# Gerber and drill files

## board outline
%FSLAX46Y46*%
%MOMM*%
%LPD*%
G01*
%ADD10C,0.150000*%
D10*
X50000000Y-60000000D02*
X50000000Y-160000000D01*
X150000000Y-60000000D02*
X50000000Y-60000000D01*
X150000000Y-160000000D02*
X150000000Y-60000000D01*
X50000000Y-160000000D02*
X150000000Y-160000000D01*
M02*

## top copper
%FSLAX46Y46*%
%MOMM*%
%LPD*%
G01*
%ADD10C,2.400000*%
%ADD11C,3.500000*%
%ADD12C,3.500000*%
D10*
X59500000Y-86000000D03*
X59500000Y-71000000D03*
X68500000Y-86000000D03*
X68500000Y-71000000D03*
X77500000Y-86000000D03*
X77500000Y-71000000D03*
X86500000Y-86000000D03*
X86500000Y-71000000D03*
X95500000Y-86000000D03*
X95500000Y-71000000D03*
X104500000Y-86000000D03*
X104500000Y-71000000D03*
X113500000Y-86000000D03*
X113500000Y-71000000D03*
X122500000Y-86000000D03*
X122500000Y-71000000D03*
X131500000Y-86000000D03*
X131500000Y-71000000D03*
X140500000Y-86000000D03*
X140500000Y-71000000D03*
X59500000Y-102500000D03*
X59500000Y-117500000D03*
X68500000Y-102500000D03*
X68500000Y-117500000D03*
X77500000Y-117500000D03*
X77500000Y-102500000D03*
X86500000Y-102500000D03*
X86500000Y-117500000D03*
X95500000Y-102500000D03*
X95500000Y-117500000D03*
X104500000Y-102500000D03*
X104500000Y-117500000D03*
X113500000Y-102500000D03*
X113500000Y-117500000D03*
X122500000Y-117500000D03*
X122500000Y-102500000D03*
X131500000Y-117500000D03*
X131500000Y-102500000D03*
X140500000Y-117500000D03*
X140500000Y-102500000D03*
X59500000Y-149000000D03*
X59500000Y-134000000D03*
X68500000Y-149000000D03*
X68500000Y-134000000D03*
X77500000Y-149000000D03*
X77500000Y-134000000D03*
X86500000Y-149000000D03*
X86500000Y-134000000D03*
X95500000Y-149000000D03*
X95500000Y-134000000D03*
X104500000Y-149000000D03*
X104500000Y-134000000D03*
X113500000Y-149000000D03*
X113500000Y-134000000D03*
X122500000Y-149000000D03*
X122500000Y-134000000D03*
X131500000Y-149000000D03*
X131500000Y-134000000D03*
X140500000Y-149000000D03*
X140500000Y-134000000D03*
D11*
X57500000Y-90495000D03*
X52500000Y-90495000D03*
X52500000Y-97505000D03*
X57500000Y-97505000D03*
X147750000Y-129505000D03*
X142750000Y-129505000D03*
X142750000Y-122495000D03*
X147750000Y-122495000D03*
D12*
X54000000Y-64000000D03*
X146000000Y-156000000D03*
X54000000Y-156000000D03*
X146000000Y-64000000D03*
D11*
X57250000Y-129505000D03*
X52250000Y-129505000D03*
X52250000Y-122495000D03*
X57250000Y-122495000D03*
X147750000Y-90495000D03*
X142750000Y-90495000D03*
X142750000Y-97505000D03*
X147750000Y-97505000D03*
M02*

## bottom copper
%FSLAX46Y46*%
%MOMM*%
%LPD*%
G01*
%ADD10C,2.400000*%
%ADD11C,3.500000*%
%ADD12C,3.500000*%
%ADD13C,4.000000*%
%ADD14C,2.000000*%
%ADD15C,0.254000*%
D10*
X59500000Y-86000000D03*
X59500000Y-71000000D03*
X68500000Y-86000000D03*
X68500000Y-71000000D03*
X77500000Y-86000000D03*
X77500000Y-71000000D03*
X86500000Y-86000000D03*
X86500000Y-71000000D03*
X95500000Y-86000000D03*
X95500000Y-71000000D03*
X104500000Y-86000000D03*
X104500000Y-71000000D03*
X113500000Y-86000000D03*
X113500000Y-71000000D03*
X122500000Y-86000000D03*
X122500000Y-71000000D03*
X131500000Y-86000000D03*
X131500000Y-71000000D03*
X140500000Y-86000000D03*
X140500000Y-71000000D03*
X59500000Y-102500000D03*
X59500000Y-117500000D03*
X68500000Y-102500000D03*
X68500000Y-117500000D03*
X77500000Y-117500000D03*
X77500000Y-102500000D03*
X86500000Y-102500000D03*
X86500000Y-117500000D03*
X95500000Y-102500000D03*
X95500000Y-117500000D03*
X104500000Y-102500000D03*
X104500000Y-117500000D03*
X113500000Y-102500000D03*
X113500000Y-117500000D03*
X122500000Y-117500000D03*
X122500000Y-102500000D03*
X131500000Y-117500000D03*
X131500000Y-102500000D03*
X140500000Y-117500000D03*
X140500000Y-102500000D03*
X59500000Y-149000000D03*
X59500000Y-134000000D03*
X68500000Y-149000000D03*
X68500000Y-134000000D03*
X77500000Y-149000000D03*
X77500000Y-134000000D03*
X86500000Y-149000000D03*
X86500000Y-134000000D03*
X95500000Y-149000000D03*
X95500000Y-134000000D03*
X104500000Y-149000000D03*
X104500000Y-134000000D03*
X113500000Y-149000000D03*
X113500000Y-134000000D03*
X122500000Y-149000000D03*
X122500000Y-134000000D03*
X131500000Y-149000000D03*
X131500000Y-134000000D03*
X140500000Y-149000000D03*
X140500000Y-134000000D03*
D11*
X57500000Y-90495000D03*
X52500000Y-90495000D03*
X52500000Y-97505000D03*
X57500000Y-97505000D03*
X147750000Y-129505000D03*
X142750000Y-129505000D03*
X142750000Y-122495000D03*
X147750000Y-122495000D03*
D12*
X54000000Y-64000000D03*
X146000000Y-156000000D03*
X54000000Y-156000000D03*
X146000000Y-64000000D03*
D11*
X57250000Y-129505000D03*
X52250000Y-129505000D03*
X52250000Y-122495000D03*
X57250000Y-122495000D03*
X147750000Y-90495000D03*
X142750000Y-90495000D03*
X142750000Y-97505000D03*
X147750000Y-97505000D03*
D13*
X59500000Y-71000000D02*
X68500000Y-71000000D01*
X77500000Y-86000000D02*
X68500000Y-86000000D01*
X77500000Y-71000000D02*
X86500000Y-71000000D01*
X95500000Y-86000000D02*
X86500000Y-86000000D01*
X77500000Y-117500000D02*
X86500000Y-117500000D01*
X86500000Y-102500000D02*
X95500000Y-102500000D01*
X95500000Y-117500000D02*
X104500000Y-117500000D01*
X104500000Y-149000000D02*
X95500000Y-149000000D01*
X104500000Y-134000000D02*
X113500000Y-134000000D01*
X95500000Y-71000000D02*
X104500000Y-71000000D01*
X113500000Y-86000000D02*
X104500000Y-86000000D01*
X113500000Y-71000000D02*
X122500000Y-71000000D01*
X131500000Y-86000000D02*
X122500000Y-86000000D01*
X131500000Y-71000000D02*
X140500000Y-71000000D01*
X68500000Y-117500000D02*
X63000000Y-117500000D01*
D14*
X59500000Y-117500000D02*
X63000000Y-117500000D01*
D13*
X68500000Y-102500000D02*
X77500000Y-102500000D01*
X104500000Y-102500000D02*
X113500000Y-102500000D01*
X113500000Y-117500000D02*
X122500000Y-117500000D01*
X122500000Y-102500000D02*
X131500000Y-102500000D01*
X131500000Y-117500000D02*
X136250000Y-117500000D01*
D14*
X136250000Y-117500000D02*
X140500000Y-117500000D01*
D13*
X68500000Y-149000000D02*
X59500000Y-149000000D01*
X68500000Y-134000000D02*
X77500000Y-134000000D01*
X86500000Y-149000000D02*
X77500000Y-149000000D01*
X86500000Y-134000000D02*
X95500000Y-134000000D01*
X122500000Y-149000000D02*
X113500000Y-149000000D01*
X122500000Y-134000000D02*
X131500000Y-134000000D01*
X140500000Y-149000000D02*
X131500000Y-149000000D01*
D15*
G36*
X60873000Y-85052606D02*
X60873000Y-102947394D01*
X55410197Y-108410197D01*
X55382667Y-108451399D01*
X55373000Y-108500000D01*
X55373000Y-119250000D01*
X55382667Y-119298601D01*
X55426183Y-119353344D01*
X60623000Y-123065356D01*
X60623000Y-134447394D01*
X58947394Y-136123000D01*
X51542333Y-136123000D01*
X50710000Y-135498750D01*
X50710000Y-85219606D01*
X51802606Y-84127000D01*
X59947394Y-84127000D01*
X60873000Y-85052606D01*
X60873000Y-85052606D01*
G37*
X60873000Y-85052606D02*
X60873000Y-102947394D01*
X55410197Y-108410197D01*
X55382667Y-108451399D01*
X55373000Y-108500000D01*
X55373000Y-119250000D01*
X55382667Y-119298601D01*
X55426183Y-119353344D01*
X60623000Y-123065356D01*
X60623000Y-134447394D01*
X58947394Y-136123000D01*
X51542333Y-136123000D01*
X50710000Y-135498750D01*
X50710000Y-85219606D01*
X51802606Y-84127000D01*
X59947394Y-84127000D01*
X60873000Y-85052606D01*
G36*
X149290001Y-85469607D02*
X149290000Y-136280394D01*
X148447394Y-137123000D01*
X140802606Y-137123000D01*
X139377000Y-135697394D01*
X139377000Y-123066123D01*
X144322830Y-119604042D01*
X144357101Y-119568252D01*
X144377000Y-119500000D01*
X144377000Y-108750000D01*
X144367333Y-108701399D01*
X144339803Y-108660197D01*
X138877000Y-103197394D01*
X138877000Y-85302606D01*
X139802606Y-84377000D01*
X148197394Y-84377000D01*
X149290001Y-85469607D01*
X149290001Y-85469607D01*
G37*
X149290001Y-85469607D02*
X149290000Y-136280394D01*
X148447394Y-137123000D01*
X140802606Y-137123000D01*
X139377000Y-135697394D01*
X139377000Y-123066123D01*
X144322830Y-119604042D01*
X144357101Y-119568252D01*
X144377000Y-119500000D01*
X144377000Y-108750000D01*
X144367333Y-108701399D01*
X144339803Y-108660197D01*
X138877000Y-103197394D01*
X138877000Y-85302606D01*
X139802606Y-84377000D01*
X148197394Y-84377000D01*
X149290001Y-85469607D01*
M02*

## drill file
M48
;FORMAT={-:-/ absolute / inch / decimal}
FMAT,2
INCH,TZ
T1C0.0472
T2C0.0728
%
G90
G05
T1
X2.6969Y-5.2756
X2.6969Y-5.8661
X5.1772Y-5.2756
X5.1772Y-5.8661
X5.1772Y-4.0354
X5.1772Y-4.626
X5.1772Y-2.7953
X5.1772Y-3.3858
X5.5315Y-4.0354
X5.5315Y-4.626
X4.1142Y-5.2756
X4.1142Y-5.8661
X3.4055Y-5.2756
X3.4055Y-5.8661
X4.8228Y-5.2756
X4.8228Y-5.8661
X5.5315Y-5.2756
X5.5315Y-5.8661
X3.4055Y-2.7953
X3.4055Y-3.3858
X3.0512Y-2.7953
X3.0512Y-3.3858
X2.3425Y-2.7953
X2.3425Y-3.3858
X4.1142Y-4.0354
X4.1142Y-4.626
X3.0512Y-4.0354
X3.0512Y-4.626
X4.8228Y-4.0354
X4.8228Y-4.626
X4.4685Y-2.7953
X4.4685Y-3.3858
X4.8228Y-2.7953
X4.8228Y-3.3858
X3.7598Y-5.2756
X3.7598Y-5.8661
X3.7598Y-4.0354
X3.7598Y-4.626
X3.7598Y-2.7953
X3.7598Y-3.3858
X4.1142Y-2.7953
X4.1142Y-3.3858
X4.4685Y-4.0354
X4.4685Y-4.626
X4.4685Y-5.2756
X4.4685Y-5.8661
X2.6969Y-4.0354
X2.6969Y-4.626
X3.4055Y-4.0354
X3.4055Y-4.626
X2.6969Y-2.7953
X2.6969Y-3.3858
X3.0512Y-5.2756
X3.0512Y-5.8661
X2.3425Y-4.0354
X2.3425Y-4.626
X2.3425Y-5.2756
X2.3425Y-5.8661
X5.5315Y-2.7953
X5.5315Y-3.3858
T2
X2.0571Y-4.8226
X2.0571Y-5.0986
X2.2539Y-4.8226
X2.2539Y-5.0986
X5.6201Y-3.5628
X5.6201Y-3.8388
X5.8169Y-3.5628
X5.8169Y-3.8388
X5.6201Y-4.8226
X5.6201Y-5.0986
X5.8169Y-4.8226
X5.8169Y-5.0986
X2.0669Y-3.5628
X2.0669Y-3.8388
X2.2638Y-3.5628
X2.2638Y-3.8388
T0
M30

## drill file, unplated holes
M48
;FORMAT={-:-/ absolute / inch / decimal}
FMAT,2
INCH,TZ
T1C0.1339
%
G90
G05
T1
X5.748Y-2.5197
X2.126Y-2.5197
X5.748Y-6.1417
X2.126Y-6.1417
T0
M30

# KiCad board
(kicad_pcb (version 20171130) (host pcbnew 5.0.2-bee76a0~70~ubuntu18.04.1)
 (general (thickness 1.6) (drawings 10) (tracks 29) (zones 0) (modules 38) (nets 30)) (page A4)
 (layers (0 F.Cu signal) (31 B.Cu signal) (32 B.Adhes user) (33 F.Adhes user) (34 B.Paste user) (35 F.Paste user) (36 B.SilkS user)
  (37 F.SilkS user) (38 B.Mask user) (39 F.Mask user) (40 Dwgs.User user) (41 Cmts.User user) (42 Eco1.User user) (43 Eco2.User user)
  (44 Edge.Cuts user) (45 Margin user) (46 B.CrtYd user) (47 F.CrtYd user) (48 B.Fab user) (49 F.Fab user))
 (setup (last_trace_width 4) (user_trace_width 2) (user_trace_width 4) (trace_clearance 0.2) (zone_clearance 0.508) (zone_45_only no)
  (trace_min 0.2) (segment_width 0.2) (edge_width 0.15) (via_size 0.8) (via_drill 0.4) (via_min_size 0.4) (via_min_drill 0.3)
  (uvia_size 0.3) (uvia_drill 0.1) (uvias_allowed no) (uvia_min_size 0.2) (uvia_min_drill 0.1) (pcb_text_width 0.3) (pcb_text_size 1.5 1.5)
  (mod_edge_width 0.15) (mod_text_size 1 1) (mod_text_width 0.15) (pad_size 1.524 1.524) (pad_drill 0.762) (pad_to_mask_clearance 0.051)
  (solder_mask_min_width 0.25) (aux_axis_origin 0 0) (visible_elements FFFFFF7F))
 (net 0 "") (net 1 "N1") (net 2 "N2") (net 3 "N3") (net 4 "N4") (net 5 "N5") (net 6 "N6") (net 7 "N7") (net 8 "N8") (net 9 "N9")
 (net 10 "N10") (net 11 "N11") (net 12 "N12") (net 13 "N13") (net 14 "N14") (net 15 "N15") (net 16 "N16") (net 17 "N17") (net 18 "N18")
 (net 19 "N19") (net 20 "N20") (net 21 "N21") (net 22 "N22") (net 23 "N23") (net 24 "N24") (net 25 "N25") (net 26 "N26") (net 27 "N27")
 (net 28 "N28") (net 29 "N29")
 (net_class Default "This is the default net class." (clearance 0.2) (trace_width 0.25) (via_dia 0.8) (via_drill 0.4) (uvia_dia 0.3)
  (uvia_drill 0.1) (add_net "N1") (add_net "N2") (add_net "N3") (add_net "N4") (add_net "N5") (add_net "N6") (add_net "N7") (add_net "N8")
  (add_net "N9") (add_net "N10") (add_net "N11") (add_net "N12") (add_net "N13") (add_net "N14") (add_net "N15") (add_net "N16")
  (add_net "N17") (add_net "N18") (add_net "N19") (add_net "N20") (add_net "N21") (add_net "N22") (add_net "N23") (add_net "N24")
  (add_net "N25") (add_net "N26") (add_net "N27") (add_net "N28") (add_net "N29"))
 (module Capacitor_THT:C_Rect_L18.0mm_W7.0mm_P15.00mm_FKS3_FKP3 (layer F.Cu) (at 59.5 86 90)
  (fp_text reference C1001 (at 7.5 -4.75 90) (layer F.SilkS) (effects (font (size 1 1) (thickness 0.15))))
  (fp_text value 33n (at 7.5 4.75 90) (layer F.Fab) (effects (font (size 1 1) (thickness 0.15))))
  (pad 1 thru_hole circle (at 0 0 90) (size 2.4 2.4) (drill 1.2) (layers *.Cu *.Mask) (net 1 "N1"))
  (pad 2 thru_hole circle (at 15 0 90) (size 2.4 2.4) (drill 1.2) (layers *.Cu *.Mask) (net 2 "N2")))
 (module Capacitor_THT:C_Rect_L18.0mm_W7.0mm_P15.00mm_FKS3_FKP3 (layer F.Cu) (at 68.5 71 270)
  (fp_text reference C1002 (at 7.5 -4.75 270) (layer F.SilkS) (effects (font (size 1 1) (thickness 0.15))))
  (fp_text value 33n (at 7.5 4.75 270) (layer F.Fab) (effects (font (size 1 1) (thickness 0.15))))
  (pad 2 thru_hole circle (at 15 0 270) (size 2.4 2.4) (drill 1.2) (layers *.Cu *.Mask) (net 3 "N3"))
  (pad 1 thru_hole circle (at 0 0 270) (size 2.4 2.4) (drill 1.2) (layers *.Cu *.Mask) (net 2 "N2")))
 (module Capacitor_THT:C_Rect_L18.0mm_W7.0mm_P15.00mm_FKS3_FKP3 (layer F.Cu) (at 77.5 86 90)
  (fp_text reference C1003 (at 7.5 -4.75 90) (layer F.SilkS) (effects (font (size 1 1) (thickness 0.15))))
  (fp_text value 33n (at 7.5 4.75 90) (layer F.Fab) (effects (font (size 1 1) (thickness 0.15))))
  (pad 1 thru_hole circle (at 0 0 90) (size 2.4 2.4) (drill 1.2) (layers *.Cu *.Mask) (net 3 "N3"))
  (pad 2 thru_hole circle (at 15 0 90) (size 2.4 2.4) (drill 1.2) (layers *.Cu *.Mask) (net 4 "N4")))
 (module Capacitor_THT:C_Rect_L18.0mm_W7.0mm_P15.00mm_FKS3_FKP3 (layer F.Cu) (at 86.5 71 270)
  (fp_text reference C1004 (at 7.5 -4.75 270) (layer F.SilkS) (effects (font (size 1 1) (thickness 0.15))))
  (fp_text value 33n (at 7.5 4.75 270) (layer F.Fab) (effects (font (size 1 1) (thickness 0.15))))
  (pad 2 thru_hole circle (at 15 0 270) (size 2.4 2.4) (drill 1.2) (layers *.Cu *.Mask) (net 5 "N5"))
  (pad 1 thru_hole circle (at 0 0 270) (size 2.4 2.4) (drill 1.2) (layers *.Cu *.Mask) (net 4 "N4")))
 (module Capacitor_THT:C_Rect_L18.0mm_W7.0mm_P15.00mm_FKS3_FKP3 (layer F.Cu) (at 95.5 86 90)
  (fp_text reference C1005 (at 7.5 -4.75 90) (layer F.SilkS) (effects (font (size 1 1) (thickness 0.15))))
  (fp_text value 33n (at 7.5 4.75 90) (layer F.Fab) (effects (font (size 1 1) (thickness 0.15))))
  (pad 1 thru_hole circle (at 0 0 90) (size 2.4 2.4) (drill 1.2) (layers *.Cu *.Mask) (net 5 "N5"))
  (pad 2 thru_hole circle (at 15 0 90) (size 2.4 2.4) (drill 1.2) (layers *.Cu *.Mask) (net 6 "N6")))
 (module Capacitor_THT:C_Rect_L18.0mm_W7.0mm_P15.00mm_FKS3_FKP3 (layer F.Cu) (at 104.5 71 270)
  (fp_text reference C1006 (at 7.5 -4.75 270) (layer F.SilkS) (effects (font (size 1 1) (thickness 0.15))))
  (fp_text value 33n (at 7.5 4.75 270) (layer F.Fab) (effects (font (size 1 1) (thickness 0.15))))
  (pad 2 thru_hole circle (at 15 0 270) (size 2.4 2.4) (drill 1.2) (layers *.Cu *.Mask) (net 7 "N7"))
  (pad 1 thru_hole circle (at 0 0 270) (size 2.4 2.4) (drill 1.2) (layers *.Cu *.Mask) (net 6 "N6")))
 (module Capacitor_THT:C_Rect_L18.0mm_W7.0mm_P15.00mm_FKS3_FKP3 (layer F.Cu) (at 113.5 86 90)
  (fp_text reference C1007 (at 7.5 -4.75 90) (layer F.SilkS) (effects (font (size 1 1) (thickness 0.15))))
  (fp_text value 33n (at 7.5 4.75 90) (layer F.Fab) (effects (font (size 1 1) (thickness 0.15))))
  (pad 1 thru_hole circle (at 0 0 90) (size 2.4 2.4) (drill 1.2) (layers *.Cu *.Mask) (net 7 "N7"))
  (pad 2 thru_hole circle (at 15 0 90) (size 2.4 2.4) (drill 1.2) (layers *.Cu *.Mask) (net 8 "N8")))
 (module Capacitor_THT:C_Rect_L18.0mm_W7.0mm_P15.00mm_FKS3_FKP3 (layer F.Cu) (at 122.5 71 270)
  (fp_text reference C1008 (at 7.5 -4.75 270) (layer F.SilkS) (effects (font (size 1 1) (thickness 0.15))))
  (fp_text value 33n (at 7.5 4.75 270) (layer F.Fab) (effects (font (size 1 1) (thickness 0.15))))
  (pad 2 thru_hole circle (at 15 0 270) (size 2.4 2.4) (drill 1.2) (layers *.Cu *.Mask) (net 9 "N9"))
  (pad 1 thru_hole circle (at 0 0 270) (size 2.4 2.4) (drill 1.2) (layers *.Cu *.Mask) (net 8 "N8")))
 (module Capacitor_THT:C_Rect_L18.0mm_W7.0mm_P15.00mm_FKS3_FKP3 (layer F.Cu) (at 131.5 86 90)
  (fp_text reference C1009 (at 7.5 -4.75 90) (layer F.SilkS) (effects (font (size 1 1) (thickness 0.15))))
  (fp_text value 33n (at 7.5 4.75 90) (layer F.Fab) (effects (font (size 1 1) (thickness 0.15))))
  (pad 1 thru_hole circle (at 0 0 90) (size 2.4 2.4) (drill 1.2) (layers *.Cu *.Mask) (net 9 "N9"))
  (pad 2 thru_hole circle (at 15 0 90) (size 2.4 2.4) (drill 1.2) (layers *.Cu *.Mask) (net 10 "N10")))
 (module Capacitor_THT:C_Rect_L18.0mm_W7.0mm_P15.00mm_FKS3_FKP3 (layer F.Cu) (at 140.5 71 270)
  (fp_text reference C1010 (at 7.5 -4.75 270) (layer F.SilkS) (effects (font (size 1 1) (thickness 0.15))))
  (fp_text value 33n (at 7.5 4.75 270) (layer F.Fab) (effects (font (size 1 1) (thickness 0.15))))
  (pad 2 thru_hole circle (at 15 0 270) (size 2.4 2.4) (drill 1.2) (layers *.Cu *.Mask) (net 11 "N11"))
  (pad 1 thru_hole circle (at 0 0 270) (size 2.4 2.4) (drill 1.2) (layers *.Cu *.Mask) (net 10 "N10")))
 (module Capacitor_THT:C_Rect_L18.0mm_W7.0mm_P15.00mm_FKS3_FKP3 (layer F.Cu) (at 59.5 102.5 270)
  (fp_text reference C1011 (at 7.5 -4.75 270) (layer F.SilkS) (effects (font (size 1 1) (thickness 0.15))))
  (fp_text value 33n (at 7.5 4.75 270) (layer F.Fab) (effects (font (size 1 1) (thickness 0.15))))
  (pad 1 thru_hole circle (at 0 0 270) (size 2.4 2.4) (drill 1.2) (layers *.Cu *.Mask) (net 1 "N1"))
  (pad 2 thru_hole circle (at 15 0 270) (size 2.4 2.4) (drill 1.2) (layers *.Cu *.Mask) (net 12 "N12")))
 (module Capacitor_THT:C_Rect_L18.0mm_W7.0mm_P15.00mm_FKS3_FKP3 (layer F.Cu) (at 68.5 117.5 90)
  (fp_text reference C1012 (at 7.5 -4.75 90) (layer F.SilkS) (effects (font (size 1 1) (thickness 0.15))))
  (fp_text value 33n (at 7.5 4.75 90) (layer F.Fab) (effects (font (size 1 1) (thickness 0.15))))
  (pad 2 thru_hole circle (at 15 0 90) (size 2.4 2.4) (drill 1.2) (layers *.Cu *.Mask) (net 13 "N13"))
  (pad 1 thru_hole circle (at 0 0 90) (size 2.4 2.4) (drill 1.2) (layers *.Cu *.Mask) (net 12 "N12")))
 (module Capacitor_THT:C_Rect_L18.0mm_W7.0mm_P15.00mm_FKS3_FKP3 (layer F.Cu) (at 77.5 102.5 270)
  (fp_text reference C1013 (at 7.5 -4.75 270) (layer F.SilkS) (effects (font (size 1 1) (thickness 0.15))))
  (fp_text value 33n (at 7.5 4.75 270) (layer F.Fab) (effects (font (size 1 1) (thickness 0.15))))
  (pad 2 thru_hole circle (at 15 0 270) (size 2.4 2.4) (drill 1.2) (layers *.Cu *.Mask) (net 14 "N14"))
  (pad 1 thru_hole circle (at 0 0 270) (size 2.4 2.4) (drill 1.2) (layers *.Cu *.Mask) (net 13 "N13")))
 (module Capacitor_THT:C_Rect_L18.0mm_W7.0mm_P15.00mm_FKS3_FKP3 (layer F.Cu) (at 86.5 117.5 90)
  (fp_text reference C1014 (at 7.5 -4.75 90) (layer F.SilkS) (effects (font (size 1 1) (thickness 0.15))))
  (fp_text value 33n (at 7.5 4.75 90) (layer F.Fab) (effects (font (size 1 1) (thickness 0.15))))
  (pad 2 thru_hole circle (at 15 0 90) (size 2.4 2.4) (drill 1.2) (layers *.Cu *.Mask) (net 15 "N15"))
  (pad 1 thru_hole circle (at 0 0 90) (size 2.4 2.4) (drill 1.2) (layers *.Cu *.Mask) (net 14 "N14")))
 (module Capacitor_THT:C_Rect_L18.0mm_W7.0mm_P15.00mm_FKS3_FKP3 (layer F.Cu) (at 95.5 102.5 270)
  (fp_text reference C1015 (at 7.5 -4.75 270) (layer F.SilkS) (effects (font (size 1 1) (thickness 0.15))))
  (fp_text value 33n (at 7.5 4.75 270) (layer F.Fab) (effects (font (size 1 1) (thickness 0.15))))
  (pad 1 thru_hole circle (at 0 0 270) (size 2.4 2.4) (drill 1.2) (layers *.Cu *.Mask) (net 15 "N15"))
  (pad 2 thru_hole circle (at 15 0 270) (size 2.4 2.4) (drill 1.2) (layers *.Cu *.Mask) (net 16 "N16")))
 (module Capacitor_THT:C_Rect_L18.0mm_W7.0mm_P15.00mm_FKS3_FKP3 (layer F.Cu) (at 104.5 117.5 90)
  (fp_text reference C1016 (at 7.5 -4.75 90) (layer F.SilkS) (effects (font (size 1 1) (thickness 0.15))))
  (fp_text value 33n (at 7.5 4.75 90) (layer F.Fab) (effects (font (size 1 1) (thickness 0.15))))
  (pad 2 thru_hole circle (at 15 0 90) (size 2.4 2.4) (drill 1.2) (layers *.Cu *.Mask) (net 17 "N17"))
  (pad 1 thru_hole circle (at 0 0 90) (size 2.4 2.4) (drill 1.2) (layers *.Cu *.Mask) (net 16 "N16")))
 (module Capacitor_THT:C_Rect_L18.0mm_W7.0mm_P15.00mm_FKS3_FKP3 (layer F.Cu) (at 113.5 102.5 270)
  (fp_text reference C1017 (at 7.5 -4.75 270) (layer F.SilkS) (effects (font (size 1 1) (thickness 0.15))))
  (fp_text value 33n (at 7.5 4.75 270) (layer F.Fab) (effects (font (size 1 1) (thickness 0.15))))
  (pad 1 thru_hole circle (at 0 0 270) (size 2.4 2.4) (drill 1.2) (layers *.Cu *.Mask) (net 17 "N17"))
  (pad 2 thru_hole circle (at 15 0 270) (size 2.4 2.4) (drill 1.2) (layers *.Cu *.Mask) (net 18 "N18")))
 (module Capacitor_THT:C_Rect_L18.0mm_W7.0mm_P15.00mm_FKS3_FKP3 (layer F.Cu) (at 122.5 117.5 90)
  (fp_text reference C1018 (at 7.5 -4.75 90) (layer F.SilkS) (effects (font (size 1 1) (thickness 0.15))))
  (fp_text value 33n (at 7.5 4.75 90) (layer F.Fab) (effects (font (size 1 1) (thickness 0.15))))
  (pad 1 thru_hole circle (at 0 0 90) (size 2.4 2.4) (drill 1.2) (layers *.Cu *.Mask) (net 18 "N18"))
  (pad 2 thru_hole circle (at 15 0 90) (size 2.4 2.4) (drill 1.2) (layers *.Cu *.Mask) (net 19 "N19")))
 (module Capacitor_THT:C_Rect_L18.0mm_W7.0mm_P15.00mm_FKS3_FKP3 (layer F.Cu) (at 131.5 102.5 270)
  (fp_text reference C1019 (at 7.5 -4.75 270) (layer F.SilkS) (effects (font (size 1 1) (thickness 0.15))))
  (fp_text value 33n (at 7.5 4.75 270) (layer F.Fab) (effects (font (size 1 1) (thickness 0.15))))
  (pad 2 thru_hole circle (at 15 0 270) (size 2.4 2.4) (drill 1.2) (layers *.Cu *.Mask) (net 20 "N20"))
  (pad 1 thru_hole circle (at 0 0 270) (size 2.4 2.4) (drill 1.2) (layers *.Cu *.Mask) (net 19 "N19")))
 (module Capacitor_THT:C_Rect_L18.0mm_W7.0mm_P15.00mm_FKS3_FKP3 (layer F.Cu) (at 140.5 117.5 90)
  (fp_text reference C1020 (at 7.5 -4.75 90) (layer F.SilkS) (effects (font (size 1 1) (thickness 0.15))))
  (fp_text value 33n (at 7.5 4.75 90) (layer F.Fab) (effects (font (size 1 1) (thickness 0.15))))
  (pad 1 thru_hole circle (at 0 0 90) (size 2.4 2.4) (drill 1.2) (layers *.Cu *.Mask) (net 20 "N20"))
  (pad 2 thru_hole circle (at 15 0 90) (size 2.4 2.4) (drill 1.2) (layers *.Cu *.Mask) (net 11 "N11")))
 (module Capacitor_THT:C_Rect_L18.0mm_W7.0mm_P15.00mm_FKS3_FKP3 (layer F.Cu) (at 59.5 134 270)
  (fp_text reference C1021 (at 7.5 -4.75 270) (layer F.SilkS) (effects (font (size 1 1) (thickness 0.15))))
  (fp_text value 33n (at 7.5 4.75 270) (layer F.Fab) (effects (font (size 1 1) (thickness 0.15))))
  (pad 2 thru_hole circle (at 15 0 270) (size 2.4 2.4) (drill 1.2) (layers *.Cu *.Mask) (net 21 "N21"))
  (pad 1 thru_hole circle (at 0 0 270) (size 2.4 2.4) (drill 1.2) (layers *.Cu *.Mask) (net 1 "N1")))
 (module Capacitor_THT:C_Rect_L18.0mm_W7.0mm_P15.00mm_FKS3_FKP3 (layer F.Cu) (at 68.5 149 90)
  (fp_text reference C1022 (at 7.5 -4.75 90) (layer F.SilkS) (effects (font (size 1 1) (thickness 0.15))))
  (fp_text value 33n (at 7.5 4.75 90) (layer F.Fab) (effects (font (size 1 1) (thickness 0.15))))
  (pad 1 thru_hole circle (at 0 0 90) (size 2.4 2.4) (drill 1.2) (layers *.Cu *.Mask) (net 21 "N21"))
  (pad 2 thru_hole circle (at 15 0 90) (size 2.4 2.4) (drill 1.2) (layers *.Cu *.Mask) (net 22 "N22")))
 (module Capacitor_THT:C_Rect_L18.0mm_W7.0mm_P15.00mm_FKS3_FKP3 (layer F.Cu) (at 77.5 134 270)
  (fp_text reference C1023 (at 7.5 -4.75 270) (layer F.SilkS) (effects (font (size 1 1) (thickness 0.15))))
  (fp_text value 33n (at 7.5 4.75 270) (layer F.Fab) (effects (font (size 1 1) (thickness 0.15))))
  (pad 2 thru_hole circle (at 15 0 270) (size 2.4 2.4) (drill 1.2) (layers *.Cu *.Mask) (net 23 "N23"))
  (pad 1 thru_hole circle (at 0 0 270) (size 2.4 2.4) (drill 1.2) (layers *.Cu *.Mask) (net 22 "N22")))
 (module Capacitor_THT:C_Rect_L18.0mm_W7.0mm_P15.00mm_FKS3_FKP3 (layer F.Cu) (at 86.5 149 90)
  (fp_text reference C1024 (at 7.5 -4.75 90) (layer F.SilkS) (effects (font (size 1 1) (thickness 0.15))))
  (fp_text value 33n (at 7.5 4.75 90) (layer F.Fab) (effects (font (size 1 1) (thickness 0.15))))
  (pad 1 thru_hole circle (at 0 0 90) (size 2.4 2.4) (drill 1.2) (layers *.Cu *.Mask) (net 23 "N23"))
  (pad 2 thru_hole circle (at 15 0 90) (size 2.4 2.4) (drill 1.2) (layers *.Cu *.Mask) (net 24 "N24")))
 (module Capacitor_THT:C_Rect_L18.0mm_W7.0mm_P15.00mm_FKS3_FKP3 (layer F.Cu) (at 95.5 134 270)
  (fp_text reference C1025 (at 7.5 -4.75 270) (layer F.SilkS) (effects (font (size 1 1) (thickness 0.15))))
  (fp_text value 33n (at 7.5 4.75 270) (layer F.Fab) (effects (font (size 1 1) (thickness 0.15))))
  (pad 2 thru_hole circle (at 15 0 270) (size 2.4 2.4) (drill 1.2) (layers *.Cu *.Mask) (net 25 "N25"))
  (pad 1 thru_hole circle (at 0 0 270) (size 2.4 2.4) (drill 1.2) (layers *.Cu *.Mask) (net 24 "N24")))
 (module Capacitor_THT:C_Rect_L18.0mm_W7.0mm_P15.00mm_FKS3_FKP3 (layer F.Cu) (at 104.5 149 90)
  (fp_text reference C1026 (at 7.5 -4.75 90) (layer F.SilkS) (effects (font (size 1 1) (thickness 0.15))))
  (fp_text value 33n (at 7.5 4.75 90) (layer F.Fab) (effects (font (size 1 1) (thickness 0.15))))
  (pad 1 thru_hole circle (at 0 0 90) (size 2.4 2.4) (drill 1.2) (layers *.Cu *.Mask) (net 25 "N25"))
  (pad 2 thru_hole circle (at 15 0 90) (size 2.4 2.4) (drill 1.2) (layers *.Cu *.Mask) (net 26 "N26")))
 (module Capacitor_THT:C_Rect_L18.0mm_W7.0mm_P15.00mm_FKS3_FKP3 (layer F.Cu) (at 113.5 134 270)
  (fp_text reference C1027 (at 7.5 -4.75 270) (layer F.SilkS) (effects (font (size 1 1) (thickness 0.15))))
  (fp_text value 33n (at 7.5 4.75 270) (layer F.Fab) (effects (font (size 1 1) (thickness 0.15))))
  (pad 2 thru_hole circle (at 15 0 270) (size 2.4 2.4) (drill 1.2) (layers *.Cu *.Mask) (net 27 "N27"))
  (pad 1 thru_hole circle (at 0 0 270) (size 2.4 2.4) (drill 1.2) (layers *.Cu *.Mask) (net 26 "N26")))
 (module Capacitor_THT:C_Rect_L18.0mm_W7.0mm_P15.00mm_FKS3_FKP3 (layer F.Cu) (at 122.5 149 90)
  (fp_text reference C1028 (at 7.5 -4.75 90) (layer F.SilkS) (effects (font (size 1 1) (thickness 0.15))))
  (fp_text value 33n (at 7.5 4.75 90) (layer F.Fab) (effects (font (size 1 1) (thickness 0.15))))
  (pad 1 thru_hole circle (at 0 0 90) (size 2.4 2.4) (drill 1.2) (layers *.Cu *.Mask) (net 27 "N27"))
  (pad 2 thru_hole circle (at 15 0 90) (size 2.4 2.4) (drill 1.2) (layers *.Cu *.Mask) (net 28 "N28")))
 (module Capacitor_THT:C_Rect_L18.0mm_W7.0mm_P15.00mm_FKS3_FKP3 (layer F.Cu) (at 131.5 134 270)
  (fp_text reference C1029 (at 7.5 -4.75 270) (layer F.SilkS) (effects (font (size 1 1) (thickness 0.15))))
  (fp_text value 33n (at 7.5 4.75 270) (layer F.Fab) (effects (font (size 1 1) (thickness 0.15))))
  (pad 2 thru_hole circle (at 15 0 270) (size 2.4 2.4) (drill 1.2) (layers *.Cu *.Mask) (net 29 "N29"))
  (pad 1 thru_hole circle (at 0 0 270) (size 2.4 2.4) (drill 1.2) (layers *.Cu *.Mask) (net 28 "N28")))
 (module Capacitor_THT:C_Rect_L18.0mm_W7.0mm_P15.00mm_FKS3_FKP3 (layer F.Cu) (at 140.5 149 90)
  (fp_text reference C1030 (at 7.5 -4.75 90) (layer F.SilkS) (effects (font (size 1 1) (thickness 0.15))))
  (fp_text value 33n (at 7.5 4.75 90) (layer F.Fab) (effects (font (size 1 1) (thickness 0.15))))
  (pad 1 thru_hole circle (at 0 0 90) (size 2.4 2.4) (drill 1.2) (layers *.Cu *.Mask) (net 29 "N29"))
  (pad 2 thru_hole circle (at 15 0 90) (size 2.4 2.4) (drill 1.2) (layers *.Cu *.Mask) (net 11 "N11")))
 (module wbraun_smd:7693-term (layer F.Cu) (at 55 94)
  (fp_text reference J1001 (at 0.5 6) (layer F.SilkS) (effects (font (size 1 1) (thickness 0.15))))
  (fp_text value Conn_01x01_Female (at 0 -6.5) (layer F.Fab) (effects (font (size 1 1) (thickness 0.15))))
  (pad 1 thru_hole circle (at 2.5 -3.505) (size 3.5 3.5) (drill 1.85) (layers *.Cu *.Mask) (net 1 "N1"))
  (pad 1 thru_hole circle (at -2.5 -3.505) (size 3.5 3.5) (drill 1.85) (layers *.Cu *.Mask) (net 1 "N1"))
  (pad 1 thru_hole circle (at -2.5 3.505) (size 3.5 3.5) (drill 1.85) (layers *.Cu *.Mask) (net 1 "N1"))
  (pad 1 thru_hole circle (at 2.5 3.505) (size 3.5 3.5) (drill 1.85) (layers *.Cu *.Mask) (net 1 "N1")))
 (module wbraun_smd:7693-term (layer F.Cu) (at 145.25 126)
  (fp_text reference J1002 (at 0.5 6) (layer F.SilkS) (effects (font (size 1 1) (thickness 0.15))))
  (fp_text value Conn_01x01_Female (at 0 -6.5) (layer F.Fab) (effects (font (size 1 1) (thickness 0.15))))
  (pad 1 thru_hole circle (at 2.5 3.505) (size 3.5 3.5) (drill 1.85) (layers *.Cu *.Mask) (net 11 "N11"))
  (pad 1 thru_hole circle (at -2.5 3.505) (size 3.5 3.5) (drill 1.85) (layers *.Cu *.Mask) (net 11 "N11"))
  (pad 1 thru_hole circle (at -2.5 -3.505) (size 3.5 3.5) (drill 1.85) (layers *.Cu *.Mask) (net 11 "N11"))
  (pad 1 thru_hole circle (at 2.5 -3.505) (size 3.5 3.5) (drill 1.85) (layers *.Cu *.Mask) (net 11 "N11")))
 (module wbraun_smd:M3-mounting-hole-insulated (layer F.Cu) (at 54 64)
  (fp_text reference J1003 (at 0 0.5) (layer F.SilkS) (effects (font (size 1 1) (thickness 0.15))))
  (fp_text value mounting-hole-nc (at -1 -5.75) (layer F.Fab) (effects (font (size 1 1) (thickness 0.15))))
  (pad "" np_thru_hole circle (at 0 0) (size 3.5 3.5) (drill 3.4) (layers *.Cu *.Mask)))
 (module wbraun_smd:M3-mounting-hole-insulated (layer F.Cu) (at 146 156)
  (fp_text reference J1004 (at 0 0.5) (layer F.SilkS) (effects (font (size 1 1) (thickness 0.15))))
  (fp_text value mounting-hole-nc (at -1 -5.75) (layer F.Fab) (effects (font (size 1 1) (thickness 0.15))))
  (pad "" np_thru_hole circle (at 0 0) (size 3.5 3.5) (drill 3.4) (layers *.Cu *.Mask)))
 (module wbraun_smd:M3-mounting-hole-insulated (layer F.Cu) (at 54 156)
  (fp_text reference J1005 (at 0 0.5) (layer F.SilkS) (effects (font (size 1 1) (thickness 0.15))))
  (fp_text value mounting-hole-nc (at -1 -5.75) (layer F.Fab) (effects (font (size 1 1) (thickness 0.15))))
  (pad "" np_thru_hole circle (at 0 0) (size 3.5 3.5) (drill 3.4) (layers *.Cu *.Mask)))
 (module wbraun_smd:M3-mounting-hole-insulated (layer F.Cu) (at 146 64)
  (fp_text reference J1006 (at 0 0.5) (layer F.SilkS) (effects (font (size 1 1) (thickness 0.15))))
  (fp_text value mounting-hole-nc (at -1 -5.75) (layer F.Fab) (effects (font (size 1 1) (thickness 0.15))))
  (pad "" np_thru_hole circle (at 0 0) (size 3.5 3.5) (drill 3.4) (layers *.Cu *.Mask)))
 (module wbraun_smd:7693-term (layer F.Cu) (at 54.75 126)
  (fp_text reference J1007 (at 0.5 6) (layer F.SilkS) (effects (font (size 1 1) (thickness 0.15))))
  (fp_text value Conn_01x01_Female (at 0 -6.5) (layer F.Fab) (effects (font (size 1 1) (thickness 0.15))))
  (pad 1 thru_hole circle (at 2.5 3.505) (size 3.5 3.5) (drill 1.85) (layers *.Cu *.Mask) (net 1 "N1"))
  (pad 1 thru_hole circle (at -2.5 3.505) (size 3.5 3.5) (drill 1.85) (layers *.Cu *.Mask) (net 1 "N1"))
  (pad 1 thru_hole circle (at -2.5 -3.505) (size 3.5 3.5) (drill 1.85) (layers *.Cu *.Mask) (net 1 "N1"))
  (pad 1 thru_hole circle (at 2.5 -3.505) (size 3.5 3.5) (drill 1.85) (layers *.Cu *.Mask) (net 1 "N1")))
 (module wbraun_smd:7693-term (layer F.Cu) (at 145.25 94)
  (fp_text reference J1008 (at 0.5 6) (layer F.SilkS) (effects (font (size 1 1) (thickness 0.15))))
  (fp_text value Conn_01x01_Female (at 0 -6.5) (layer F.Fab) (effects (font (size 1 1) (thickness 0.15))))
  (pad 1 thru_hole circle (at 2.5 -3.505) (size 3.5 3.5) (drill 1.85) (layers *.Cu *.Mask) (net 11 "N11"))
  (pad 1 thru_hole circle (at -2.5 -3.505) (size 3.5 3.5) (drill 1.85) (layers *.Cu *.Mask) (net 11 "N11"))
  (pad 1 thru_hole circle (at -2.5 3.505) (size 3.5 3.5) (drill 1.85) (layers *.Cu *.Mask) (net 11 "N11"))
  (pad 1 thru_hole circle (at 2.5 3.505) (size 3.5 3.5) (drill 1.85) (layers *.Cu *.Mask) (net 11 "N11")))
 (gr_line (start 50 60) (end 50 160) (layer Edge.Cuts) (width 0.15))
 (gr_line (start 150 60) (end 50 60) (layer Edge.Cuts) (width 0.15))
 (gr_line (start 150 160) (end 150 60) (layer Edge.Cuts) (width 0.15))
 (gr_line (start 50 160) (end 150 160) (layer Edge.Cuts) (width 0.15))
 (segment (start 59.5 71) (end 68.5 71) (width 4) (layer B.Cu) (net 2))
 (segment (start 77.5 86) (end 68.5 86) (width 4) (layer B.Cu) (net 3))
 (segment (start 77.5 71) (end 86.5 71) (width 4) (layer B.Cu) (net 4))
 (segment (start 95.5 86) (end 86.5 86) (width 4) (layer B.Cu) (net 5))
 (segment (start 77.5 117.5) (end 86.5 117.5) (width 4) (layer B.Cu) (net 14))
 (segment (start 86.5 102.5) (end 95.5 102.5) (width 4) (layer B.Cu) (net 15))
 (segment (start 95.5 117.5) (end 104.5 117.5) (width 4) (layer B.Cu) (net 16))
 (segment (start 104.5 149) (end 95.5 149) (width 4) (layer B.Cu) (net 25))
 (segment (start 104.5 134) (end 113.5 134) (width 4) (layer B.Cu) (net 26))
 (segment (start 95.5 71) (end 104.5 71) (width 4) (layer B.Cu) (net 6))
 (segment (start 113.5 86) (end 104.5 86) (width 4) (layer B.Cu) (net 7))
 (segment (start 113.5 71) (end 122.5 71) (width 4) (layer B.Cu) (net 8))
 (segment (start 131.5 86) (end 122.5 86) (width 4) (layer B.Cu) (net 9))
 (segment (start 131.5 71) (end 140.5 71) (width 4) (layer B.Cu) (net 10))
 (segment (start 68.5 117.5) (end 63 117.5) (width 4) (layer B.Cu) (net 12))
 (segment (start 59.5 117.5) (end 63 117.5) (width 2) (layer B.Cu) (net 12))
 (segment (start 68.5 102.5) (end 77.5 102.5) (width 4) (layer B.Cu) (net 13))
 (segment (start 104.5 102.5) (end 113.5 102.5) (width 4) (layer B.Cu) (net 17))
 (segment (start 113.5 117.5) (end 122.5 117.5) (width 4) (layer B.Cu) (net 18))
 (segment (start 122.5 102.5) (end 131.5 102.5) (width 4) (layer B.Cu) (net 19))
 (segment (start 131.5 117.5) (end 136.25 117.5) (width 4) (layer B.Cu) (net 20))
 (segment (start 136.25 117.5) (end 140.5 117.5) (width 2) (layer B.Cu) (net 20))
 (segment (start 68.5 149) (end 59.5 149) (width 4) (layer B.Cu) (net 21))
 (segment (start 68.5 134) (end 77.5 134) (width 4) (layer B.Cu) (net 22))
 (segment (start 86.5 149) (end 77.5 149) (width 4) (layer B.Cu) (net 23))
 (segment (start 86.5 134) (end 95.5 134) (width 4) (layer B.Cu) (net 24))
 (segment (start 122.5 149) (end 113.5 149) (width 4) (layer B.Cu) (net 27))
 (segment (start 122.5 134) (end 131.5 134) (width 4) (layer B.Cu) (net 28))
 (segment (start 140.5 149) (end 131.5 149) (width 4) (layer B.Cu) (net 29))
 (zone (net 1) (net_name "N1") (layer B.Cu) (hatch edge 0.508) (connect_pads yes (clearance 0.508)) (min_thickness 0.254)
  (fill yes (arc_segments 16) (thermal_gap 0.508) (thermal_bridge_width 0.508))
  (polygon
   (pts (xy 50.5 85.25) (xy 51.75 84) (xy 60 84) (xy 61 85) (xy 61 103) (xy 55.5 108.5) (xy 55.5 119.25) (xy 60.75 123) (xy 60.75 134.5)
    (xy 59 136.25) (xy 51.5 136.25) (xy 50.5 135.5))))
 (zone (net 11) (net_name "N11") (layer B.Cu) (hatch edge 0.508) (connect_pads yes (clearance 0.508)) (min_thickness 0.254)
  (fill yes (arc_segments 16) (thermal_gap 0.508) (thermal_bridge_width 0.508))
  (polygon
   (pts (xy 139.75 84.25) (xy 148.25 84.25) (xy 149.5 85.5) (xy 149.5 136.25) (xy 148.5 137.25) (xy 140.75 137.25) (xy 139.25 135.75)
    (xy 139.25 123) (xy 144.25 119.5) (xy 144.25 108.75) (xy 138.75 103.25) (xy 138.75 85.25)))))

